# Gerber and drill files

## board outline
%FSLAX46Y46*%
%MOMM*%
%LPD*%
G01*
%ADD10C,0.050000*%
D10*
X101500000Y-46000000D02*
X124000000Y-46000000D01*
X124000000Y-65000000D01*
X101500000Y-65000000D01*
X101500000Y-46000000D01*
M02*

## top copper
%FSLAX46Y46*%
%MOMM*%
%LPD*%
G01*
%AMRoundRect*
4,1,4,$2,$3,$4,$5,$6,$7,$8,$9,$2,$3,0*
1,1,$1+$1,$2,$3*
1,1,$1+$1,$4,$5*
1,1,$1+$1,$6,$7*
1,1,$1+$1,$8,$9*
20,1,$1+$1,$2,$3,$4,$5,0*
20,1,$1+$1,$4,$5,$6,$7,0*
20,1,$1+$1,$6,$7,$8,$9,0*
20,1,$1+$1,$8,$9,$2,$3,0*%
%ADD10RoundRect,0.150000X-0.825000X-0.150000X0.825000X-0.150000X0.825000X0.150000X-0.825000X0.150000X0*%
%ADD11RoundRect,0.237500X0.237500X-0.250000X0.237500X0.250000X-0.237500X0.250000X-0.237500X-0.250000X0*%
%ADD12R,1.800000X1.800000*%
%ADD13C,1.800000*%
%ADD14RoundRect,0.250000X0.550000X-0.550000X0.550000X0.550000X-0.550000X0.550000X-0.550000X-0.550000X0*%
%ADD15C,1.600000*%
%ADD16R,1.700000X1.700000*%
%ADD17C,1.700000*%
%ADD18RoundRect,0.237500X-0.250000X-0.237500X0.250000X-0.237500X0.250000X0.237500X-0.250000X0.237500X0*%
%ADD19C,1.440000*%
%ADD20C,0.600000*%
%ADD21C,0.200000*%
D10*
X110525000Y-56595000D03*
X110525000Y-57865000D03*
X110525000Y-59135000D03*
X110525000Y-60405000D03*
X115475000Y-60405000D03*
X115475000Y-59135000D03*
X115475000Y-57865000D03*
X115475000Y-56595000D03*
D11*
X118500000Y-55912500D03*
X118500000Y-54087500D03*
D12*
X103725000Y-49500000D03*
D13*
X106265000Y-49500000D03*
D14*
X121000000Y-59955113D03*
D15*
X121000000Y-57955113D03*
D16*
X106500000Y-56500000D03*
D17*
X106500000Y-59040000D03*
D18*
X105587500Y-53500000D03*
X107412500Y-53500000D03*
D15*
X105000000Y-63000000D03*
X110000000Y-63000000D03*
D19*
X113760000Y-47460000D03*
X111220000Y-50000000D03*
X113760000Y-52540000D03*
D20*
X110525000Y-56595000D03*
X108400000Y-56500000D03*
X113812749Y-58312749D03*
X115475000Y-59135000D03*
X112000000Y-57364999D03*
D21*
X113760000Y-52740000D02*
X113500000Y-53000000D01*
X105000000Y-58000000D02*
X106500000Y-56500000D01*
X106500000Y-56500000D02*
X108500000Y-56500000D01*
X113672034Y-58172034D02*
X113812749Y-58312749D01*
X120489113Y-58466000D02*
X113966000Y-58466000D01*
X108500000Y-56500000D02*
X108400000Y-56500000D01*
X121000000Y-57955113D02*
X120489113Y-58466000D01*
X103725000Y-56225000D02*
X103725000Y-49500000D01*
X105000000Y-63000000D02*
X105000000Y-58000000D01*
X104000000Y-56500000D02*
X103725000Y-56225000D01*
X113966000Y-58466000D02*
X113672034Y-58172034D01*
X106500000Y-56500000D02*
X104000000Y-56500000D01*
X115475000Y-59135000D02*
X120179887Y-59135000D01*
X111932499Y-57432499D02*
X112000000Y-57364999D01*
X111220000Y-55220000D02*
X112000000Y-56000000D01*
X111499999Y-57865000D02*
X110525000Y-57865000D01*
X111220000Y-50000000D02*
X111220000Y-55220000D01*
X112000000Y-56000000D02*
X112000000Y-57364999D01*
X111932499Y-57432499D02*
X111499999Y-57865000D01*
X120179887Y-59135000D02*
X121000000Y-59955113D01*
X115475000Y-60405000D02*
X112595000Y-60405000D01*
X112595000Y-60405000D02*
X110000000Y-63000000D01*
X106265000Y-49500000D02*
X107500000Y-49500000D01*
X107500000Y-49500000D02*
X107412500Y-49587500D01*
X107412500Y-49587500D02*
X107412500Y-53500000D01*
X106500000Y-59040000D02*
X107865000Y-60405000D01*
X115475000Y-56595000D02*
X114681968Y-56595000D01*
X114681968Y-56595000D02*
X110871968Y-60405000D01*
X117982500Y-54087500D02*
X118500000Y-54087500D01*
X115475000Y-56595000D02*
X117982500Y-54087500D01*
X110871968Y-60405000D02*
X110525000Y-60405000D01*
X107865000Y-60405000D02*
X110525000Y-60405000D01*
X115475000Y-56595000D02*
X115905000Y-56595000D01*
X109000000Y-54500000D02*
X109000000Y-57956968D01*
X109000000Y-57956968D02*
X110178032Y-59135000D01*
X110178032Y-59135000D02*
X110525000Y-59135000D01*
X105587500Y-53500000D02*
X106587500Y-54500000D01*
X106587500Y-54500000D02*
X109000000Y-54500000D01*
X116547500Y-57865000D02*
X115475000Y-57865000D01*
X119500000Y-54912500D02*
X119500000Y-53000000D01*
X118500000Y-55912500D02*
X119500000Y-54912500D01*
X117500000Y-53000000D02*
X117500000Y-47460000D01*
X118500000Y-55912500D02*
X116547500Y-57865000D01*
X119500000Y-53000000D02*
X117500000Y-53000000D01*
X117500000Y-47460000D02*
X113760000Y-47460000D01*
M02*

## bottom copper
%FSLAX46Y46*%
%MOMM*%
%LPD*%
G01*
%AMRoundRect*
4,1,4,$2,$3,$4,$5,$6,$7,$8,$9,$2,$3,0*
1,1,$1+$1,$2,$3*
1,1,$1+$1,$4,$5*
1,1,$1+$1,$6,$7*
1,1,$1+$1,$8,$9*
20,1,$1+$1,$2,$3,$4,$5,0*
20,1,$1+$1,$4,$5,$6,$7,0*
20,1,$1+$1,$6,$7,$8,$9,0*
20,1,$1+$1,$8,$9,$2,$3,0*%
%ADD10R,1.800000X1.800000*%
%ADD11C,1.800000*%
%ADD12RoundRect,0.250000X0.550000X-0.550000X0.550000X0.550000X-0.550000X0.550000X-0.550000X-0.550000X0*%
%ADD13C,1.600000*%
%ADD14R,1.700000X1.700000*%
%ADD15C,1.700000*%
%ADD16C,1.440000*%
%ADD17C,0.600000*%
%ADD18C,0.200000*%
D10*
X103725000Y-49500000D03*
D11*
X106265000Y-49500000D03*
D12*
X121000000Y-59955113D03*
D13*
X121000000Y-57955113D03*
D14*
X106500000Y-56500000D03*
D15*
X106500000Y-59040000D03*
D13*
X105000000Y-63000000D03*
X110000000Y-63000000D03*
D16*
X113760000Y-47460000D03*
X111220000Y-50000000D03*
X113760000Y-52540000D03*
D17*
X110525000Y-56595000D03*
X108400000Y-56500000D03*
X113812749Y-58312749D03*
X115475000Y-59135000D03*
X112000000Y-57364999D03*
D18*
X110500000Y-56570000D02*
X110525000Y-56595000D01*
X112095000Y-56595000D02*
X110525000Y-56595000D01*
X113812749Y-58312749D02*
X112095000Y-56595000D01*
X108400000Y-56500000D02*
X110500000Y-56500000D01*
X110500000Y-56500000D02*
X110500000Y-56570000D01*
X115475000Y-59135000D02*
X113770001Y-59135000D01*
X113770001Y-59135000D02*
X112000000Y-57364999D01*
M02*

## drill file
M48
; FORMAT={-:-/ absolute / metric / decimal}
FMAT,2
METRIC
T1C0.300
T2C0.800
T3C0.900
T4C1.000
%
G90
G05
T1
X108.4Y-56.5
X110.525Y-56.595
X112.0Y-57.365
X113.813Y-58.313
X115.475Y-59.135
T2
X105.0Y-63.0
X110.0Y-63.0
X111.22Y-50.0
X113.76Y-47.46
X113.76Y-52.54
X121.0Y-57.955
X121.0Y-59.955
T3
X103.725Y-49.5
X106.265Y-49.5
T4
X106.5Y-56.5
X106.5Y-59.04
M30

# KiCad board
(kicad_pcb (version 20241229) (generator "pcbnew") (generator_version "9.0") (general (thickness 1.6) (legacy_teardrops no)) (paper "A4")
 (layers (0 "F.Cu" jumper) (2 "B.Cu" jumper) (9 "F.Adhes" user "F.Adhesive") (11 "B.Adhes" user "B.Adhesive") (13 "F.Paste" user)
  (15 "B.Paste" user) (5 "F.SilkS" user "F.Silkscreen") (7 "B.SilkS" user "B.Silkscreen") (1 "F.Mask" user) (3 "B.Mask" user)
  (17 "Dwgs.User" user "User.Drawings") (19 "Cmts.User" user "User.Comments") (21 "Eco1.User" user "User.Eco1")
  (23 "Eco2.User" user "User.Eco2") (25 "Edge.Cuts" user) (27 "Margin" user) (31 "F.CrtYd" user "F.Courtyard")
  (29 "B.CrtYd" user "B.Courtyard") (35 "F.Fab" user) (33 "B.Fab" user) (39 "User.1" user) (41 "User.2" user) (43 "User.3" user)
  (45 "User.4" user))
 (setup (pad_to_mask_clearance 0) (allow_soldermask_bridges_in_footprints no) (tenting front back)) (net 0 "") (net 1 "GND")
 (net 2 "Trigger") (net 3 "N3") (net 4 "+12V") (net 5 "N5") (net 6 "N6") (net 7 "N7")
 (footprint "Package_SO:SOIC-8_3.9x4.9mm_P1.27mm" (layer "F.Cu") (at 113 58.5)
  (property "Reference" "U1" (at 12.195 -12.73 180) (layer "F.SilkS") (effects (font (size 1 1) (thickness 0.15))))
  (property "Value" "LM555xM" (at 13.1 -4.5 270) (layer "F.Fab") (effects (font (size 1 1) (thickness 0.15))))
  (pad "1" smd roundrect (at -2.475 -1.905) (size 1.95 0.6) (layers "F.Cu" "F.Mask" "F.Paste") (roundrect_rratio 0.25) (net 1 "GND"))
  (pad "2" smd roundrect (at -2.475 -0.635) (size 1.95 0.6) (layers "F.Cu" "F.Mask" "F.Paste") (roundrect_rratio 0.25) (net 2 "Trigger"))
  (pad "3" smd roundrect (at -2.475 0.635) (size 1.95 0.6) (layers "F.Cu" "F.Mask" "F.Paste") (roundrect_rratio 0.25) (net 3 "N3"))
  (pad "4" smd roundrect (at -2.475 1.905) (size 1.95 0.6) (layers "F.Cu" "F.Mask" "F.Paste") (roundrect_rratio 0.25) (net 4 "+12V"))
  (pad "5" smd roundrect (at 2.475 1.905) (size 1.95 0.6) (layers "F.Cu" "F.Mask" "F.Paste") (roundrect_rratio 0.25) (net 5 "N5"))
  (pad "6" smd roundrect (at 2.475 0.635) (size 1.95 0.6) (layers "F.Cu" "F.Mask" "F.Paste") (roundrect_rratio 0.25) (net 2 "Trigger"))
  (pad "7" smd roundrect (at 2.475 -0.635) (size 1.95 0.6) (layers "F.Cu" "F.Mask" "F.Paste") (roundrect_rratio 0.25) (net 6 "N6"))
  (pad "8" smd roundrect (at 2.475 -1.905) (size 1.95 0.6) (layers "F.Cu" "F.Mask" "F.Paste") (roundrect_rratio 0.25) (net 4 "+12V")))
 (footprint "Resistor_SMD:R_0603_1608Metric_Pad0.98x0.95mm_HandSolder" (layer "F.Cu") (at 118.5 55 90)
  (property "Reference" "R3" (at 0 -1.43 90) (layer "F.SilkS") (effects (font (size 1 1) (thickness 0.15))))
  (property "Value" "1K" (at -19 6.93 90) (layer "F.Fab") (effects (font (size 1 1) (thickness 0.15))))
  (pad "1" smd roundrect (at -0.9125 0 90) (size 0.975 0.95) (layers "F.Cu" "F.Mask" "F.Paste") (roundrect_rratio 0.25) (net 6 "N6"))
  (pad "2" smd roundrect (at 0.9125 0 90) (size 0.975 0.95) (layers "F.Cu" "F.Mask" "F.Paste") (roundrect_rratio 0.25) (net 4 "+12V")))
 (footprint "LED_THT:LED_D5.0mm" (layer "F.Cu") (at 103.725 49.5)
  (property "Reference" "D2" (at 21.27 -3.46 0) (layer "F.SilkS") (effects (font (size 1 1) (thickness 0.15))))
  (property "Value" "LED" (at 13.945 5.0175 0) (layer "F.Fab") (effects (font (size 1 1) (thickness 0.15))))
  (pad "1" thru_hole rect (at 0 0) (size 1.8 1.8) (drill 0.9) (layers "*.Cu" "*.Mask") (remove_unused_layers no) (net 1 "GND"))
  (pad "2" thru_hole circle (at 2.54 0) (size 1.8 1.8) (drill 0.9) (layers "*.Cu" "*.Mask") (remove_unused_layers no) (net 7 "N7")))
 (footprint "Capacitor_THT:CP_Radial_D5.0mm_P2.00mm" (layer "F.Cu") (at 121 59.955113 90)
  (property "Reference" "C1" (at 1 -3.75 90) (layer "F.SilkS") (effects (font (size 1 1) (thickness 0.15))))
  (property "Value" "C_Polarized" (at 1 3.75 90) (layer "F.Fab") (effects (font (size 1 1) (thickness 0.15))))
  (pad "1" thru_hole roundrect (at 0 0 90) (size 1.6 1.6) (drill 0.8) (layers "*.Cu" "*.Mask") (remove_unused_layers no)
   (roundrect_rratio 0.15625) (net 2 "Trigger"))
  (pad "2" thru_hole circle (at 2 0 90) (size 1.6 1.6) (drill 0.8) (layers "*.Cu" "*.Mask") (remove_unused_layers no) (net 1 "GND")))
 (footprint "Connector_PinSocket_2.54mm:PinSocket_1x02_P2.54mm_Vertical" (layer "F.Cu") (at 106.5 56.5)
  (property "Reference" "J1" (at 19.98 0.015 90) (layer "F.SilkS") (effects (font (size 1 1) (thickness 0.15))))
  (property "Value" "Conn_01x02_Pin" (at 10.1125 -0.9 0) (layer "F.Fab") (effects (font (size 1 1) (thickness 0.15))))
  (pad "1" thru_hole rect (at 0 0) (size 1.7 1.7) (drill 1) (layers "*.Cu" "*.Mask") (remove_unused_layers no) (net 1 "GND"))
  (pad "2" thru_hole circle (at 0 2.54) (size 1.7 1.7) (drill 1) (layers "*.Cu" "*.Mask") (remove_unused_layers no) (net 4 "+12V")))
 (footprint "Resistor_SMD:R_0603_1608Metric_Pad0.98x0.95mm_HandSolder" (layer "F.Cu") (at 106.5 53.5)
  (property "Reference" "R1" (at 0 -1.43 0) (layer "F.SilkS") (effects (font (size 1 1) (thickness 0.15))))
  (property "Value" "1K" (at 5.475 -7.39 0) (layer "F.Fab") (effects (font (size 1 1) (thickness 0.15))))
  (pad "1" smd roundrect (at -0.9125 0) (size 0.975 0.95) (layers "F.Cu" "F.Mask" "F.Paste") (roundrect_rratio 0.25) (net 3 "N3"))
  (pad "2" smd roundrect (at 0.9125 0) (size 0.975 0.95) (layers "F.Cu" "F.Mask" "F.Paste") (roundrect_rratio 0.25) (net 7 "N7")))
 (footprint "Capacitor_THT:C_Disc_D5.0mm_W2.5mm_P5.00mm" (layer "F.Cu") (at 105 63)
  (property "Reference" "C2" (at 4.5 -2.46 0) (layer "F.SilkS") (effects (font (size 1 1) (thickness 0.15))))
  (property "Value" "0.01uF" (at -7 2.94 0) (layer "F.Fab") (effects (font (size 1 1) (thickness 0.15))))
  (pad "1" thru_hole circle (at 0 0) (size 1.6 1.6) (drill 0.8) (layers "*.Cu" "*.Mask") (remove_unused_layers no) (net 1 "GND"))
  (pad "2" thru_hole circle (at 5 0) (size 1.6 1.6) (drill 0.8) (layers "*.Cu" "*.Mask") (remove_unused_layers no) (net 5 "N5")))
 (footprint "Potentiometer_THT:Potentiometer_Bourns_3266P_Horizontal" (layer "F.Cu") (at 113.76 47.46)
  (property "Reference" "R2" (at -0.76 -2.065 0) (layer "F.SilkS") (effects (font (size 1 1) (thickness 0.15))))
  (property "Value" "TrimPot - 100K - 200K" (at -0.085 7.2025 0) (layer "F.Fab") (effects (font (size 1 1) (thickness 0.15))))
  (pad "1" thru_hole circle (at 0 0) (size 1.44 1.44) (drill 0.8) (layers "*.Cu" "*.Mask") (remove_unused_layers no) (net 6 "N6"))
  (pad "2" thru_hole circle (at -2.54 2.54) (size 1.44 1.44) (drill 0.8) (layers "*.Cu" "*.Mask") (remove_unused_layers no)
   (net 2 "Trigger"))
  (pad "3" thru_hole circle (at 0 5.08) (size 1.44 1.44) (drill 0.8) (layers "*.Cu" "*.Mask") (remove_unused_layers no)))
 (gr_rect (start 101.5 46) (end 124 65) (stroke (width 0.05) (type default)) (fill no) (layer "Edge.Cuts"))
 (segment (start 113.76 52.74) (end 113.5 53) (width 0.2) (layer "F.Cu") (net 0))
 (segment (start 105 58) (end 106.5 56.5) (width 0.2) (layer "F.Cu") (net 1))
 (segment (start 106.5 56.5) (end 108.5 56.5) (width 0.2) (layer "F.Cu") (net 1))
 (segment (start 113.672034 58.172034) (end 113.812749 58.312749) (width 0.2) (layer "F.Cu") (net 1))
 (segment (start 120.489113 58.466) (end 113.966 58.466) (width 0.2) (layer "F.Cu") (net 1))
 (segment (start 108.5 56.5) (end 108.4 56.5) (width 0.2) (layer "F.Cu") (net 1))
 (segment (start 121 57.955113) (end 120.489113 58.466) (width 0.2) (layer "F.Cu") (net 1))
 (segment (start 103.725 56.225) (end 103.725 49.5) (width 0.2) (layer "F.Cu") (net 1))
 (segment (start 105 63) (end 105 58) (width 0.2) (layer "F.Cu") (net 1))
 (segment (start 104 56.5) (end 103.725 56.225) (width 0.2) (layer "F.Cu") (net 1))
 (segment (start 113.966 58.466) (end 113.672034 58.172034) (width 0.2) (layer "F.Cu") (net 1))
 (segment (start 106.5 56.5) (end 104 56.5) (width 0.2) (layer "F.Cu") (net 1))
 (via (at 110.525 56.595) (size 0.6) (drill 0.3) (layers "F.Cu" "B.Cu") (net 1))
 (via (at 108.4 56.5) (size 0.6) (drill 0.3) (layers "F.Cu" "B.Cu") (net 1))
 (via (at 113.812749 58.312749) (size 0.6) (drill 0.3) (layers "F.Cu" "B.Cu") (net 1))
 (segment (start 110.5 56.57) (end 110.525 56.595) (width 0.2) (layer "B.Cu") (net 1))
 (segment (start 112.095 56.595) (end 110.525 56.595) (width 0.2) (layer "B.Cu") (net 1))
 (segment (start 113.812749 58.312749) (end 112.095 56.595) (width 0.2) (layer "B.Cu") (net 1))
 (segment (start 108.4 56.5) (end 110.5 56.5) (width 0.2) (layer "B.Cu") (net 1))
 (segment (start 110.5 56.5) (end 110.5 56.57) (width 0.2) (layer "B.Cu") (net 1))
 (segment (start 115.475 59.135) (end 120.179887 59.135) (width 0.2) (layer "F.Cu") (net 2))
 (segment (start 111.932499 57.432499) (end 112 57.364999) (width 0.2) (layer "F.Cu") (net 2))
 (segment (start 111.22 55.22) (end 112 56) (width 0.2) (layer "F.Cu") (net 2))
 (segment (start 111.499999 57.865) (end 110.525 57.865) (width 0.2) (layer "F.Cu") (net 2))
 (segment (start 111.22 50) (end 111.22 55.22) (width 0.2) (layer "F.Cu") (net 2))
 (segment (start 112 56) (end 112 57.364999) (width 0.2) (layer "F.Cu") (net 2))
 (segment (start 111.932499 57.432499) (end 111.499999 57.865) (width 0.2) (layer "F.Cu") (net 2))
 (segment (start 120.179887 59.135) (end 121 59.955113) (width 0.2) (layer "F.Cu") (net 2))
 (via (at 115.475 59.135) (size 0.6) (drill 0.3) (layers "F.Cu" "B.Cu") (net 2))
 (via (at 112 57.364999) (size 0.6) (drill 0.3) (layers "F.Cu" "B.Cu") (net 2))
 (segment (start 115.475 59.135) (end 113.770001 59.135) (width 0.2) (layer "B.Cu") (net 2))
 (segment (start 113.770001 59.135) (end 112 57.364999) (width 0.2) (layer "B.Cu") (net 2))
 (segment (start 115.475 60.405) (end 112.595 60.405) (width 0.2) (layer "F.Cu") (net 5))
 (segment (start 112.595 60.405) (end 110 63) (width 0.2) (layer "F.Cu") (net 5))
 (segment (start 106.265 49.5) (end 107.5 49.5) (width 0.2) (layer "F.Cu") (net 7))
 (segment (start 107.5 49.5) (end 107.4125 49.5875) (width 0.2) (layer "F.Cu") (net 7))
 (segment (start 107.4125 49.5875) (end 107.4125 53.5) (width 0.2) (layer "F.Cu") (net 7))
 (segment (start 106.5 59.04) (end 107.865 60.405) (width 0.2) (layer "F.Cu") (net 4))
 (segment (start 115.475 56.595) (end 114.681968 56.595) (width 0.2) (layer "F.Cu") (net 4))
 (segment (start 114.681968 56.595) (end 110.871968 60.405) (width 0.2) (layer "F.Cu") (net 4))
 (segment (start 117.9825 54.0875) (end 118.5 54.0875) (width 0.2) (layer "F.Cu") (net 4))
 (segment (start 115.475 56.595) (end 117.9825 54.0875) (width 0.2) (layer "F.Cu") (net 4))
 (segment (start 110.871968 60.405) (end 110.525 60.405) (width 0.2) (layer "F.Cu") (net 4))
 (segment (start 107.865 60.405) (end 110.525 60.405) (width 0.2) (layer "F.Cu") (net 4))
 (segment (start 115.475 56.595) (end 115.905 56.595) (width 0.2) (layer "F.Cu") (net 4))
 (segment (start 109 54.5) (end 109 57.956968) (width 0.2) (layer "F.Cu") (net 3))
 (segment (start 109 57.956968) (end 110.178032 59.135) (width 0.2) (layer "F.Cu") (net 3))
 (segment (start 110.178032 59.135) (end 110.525 59.135) (width 0.2) (layer "F.Cu") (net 3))
 (segment (start 105.5875 53.5) (end 106.5875 54.5) (width 0.2) (layer "F.Cu") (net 3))
 (segment (start 106.5875 54.5) (end 109 54.5) (width 0.2) (layer "F.Cu") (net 3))
 (segment (start 116.5475 57.865) (end 115.475 57.865) (width 0.2) (layer "F.Cu") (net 6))
 (segment (start 119.5 54.9125) (end 119.5 53) (width 0.2) (layer "F.Cu") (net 6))
 (segment (start 118.5 55.9125) (end 119.5 54.9125) (width 0.2) (layer "F.Cu") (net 6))
 (segment (start 117.5 53) (end 117.5 47.46) (width 0.2) (layer "F.Cu") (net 6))
 (segment (start 118.5 55.9125) (end 116.5475 57.865) (width 0.2) (layer "F.Cu") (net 6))
 (segment (start 119.5 53) (end 117.5 53) (width 0.2) (layer "F.Cu") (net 6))
 (segment (start 117.5 47.46) (end 113.76 47.46) (width 0.2) (layer "F.Cu") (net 6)))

